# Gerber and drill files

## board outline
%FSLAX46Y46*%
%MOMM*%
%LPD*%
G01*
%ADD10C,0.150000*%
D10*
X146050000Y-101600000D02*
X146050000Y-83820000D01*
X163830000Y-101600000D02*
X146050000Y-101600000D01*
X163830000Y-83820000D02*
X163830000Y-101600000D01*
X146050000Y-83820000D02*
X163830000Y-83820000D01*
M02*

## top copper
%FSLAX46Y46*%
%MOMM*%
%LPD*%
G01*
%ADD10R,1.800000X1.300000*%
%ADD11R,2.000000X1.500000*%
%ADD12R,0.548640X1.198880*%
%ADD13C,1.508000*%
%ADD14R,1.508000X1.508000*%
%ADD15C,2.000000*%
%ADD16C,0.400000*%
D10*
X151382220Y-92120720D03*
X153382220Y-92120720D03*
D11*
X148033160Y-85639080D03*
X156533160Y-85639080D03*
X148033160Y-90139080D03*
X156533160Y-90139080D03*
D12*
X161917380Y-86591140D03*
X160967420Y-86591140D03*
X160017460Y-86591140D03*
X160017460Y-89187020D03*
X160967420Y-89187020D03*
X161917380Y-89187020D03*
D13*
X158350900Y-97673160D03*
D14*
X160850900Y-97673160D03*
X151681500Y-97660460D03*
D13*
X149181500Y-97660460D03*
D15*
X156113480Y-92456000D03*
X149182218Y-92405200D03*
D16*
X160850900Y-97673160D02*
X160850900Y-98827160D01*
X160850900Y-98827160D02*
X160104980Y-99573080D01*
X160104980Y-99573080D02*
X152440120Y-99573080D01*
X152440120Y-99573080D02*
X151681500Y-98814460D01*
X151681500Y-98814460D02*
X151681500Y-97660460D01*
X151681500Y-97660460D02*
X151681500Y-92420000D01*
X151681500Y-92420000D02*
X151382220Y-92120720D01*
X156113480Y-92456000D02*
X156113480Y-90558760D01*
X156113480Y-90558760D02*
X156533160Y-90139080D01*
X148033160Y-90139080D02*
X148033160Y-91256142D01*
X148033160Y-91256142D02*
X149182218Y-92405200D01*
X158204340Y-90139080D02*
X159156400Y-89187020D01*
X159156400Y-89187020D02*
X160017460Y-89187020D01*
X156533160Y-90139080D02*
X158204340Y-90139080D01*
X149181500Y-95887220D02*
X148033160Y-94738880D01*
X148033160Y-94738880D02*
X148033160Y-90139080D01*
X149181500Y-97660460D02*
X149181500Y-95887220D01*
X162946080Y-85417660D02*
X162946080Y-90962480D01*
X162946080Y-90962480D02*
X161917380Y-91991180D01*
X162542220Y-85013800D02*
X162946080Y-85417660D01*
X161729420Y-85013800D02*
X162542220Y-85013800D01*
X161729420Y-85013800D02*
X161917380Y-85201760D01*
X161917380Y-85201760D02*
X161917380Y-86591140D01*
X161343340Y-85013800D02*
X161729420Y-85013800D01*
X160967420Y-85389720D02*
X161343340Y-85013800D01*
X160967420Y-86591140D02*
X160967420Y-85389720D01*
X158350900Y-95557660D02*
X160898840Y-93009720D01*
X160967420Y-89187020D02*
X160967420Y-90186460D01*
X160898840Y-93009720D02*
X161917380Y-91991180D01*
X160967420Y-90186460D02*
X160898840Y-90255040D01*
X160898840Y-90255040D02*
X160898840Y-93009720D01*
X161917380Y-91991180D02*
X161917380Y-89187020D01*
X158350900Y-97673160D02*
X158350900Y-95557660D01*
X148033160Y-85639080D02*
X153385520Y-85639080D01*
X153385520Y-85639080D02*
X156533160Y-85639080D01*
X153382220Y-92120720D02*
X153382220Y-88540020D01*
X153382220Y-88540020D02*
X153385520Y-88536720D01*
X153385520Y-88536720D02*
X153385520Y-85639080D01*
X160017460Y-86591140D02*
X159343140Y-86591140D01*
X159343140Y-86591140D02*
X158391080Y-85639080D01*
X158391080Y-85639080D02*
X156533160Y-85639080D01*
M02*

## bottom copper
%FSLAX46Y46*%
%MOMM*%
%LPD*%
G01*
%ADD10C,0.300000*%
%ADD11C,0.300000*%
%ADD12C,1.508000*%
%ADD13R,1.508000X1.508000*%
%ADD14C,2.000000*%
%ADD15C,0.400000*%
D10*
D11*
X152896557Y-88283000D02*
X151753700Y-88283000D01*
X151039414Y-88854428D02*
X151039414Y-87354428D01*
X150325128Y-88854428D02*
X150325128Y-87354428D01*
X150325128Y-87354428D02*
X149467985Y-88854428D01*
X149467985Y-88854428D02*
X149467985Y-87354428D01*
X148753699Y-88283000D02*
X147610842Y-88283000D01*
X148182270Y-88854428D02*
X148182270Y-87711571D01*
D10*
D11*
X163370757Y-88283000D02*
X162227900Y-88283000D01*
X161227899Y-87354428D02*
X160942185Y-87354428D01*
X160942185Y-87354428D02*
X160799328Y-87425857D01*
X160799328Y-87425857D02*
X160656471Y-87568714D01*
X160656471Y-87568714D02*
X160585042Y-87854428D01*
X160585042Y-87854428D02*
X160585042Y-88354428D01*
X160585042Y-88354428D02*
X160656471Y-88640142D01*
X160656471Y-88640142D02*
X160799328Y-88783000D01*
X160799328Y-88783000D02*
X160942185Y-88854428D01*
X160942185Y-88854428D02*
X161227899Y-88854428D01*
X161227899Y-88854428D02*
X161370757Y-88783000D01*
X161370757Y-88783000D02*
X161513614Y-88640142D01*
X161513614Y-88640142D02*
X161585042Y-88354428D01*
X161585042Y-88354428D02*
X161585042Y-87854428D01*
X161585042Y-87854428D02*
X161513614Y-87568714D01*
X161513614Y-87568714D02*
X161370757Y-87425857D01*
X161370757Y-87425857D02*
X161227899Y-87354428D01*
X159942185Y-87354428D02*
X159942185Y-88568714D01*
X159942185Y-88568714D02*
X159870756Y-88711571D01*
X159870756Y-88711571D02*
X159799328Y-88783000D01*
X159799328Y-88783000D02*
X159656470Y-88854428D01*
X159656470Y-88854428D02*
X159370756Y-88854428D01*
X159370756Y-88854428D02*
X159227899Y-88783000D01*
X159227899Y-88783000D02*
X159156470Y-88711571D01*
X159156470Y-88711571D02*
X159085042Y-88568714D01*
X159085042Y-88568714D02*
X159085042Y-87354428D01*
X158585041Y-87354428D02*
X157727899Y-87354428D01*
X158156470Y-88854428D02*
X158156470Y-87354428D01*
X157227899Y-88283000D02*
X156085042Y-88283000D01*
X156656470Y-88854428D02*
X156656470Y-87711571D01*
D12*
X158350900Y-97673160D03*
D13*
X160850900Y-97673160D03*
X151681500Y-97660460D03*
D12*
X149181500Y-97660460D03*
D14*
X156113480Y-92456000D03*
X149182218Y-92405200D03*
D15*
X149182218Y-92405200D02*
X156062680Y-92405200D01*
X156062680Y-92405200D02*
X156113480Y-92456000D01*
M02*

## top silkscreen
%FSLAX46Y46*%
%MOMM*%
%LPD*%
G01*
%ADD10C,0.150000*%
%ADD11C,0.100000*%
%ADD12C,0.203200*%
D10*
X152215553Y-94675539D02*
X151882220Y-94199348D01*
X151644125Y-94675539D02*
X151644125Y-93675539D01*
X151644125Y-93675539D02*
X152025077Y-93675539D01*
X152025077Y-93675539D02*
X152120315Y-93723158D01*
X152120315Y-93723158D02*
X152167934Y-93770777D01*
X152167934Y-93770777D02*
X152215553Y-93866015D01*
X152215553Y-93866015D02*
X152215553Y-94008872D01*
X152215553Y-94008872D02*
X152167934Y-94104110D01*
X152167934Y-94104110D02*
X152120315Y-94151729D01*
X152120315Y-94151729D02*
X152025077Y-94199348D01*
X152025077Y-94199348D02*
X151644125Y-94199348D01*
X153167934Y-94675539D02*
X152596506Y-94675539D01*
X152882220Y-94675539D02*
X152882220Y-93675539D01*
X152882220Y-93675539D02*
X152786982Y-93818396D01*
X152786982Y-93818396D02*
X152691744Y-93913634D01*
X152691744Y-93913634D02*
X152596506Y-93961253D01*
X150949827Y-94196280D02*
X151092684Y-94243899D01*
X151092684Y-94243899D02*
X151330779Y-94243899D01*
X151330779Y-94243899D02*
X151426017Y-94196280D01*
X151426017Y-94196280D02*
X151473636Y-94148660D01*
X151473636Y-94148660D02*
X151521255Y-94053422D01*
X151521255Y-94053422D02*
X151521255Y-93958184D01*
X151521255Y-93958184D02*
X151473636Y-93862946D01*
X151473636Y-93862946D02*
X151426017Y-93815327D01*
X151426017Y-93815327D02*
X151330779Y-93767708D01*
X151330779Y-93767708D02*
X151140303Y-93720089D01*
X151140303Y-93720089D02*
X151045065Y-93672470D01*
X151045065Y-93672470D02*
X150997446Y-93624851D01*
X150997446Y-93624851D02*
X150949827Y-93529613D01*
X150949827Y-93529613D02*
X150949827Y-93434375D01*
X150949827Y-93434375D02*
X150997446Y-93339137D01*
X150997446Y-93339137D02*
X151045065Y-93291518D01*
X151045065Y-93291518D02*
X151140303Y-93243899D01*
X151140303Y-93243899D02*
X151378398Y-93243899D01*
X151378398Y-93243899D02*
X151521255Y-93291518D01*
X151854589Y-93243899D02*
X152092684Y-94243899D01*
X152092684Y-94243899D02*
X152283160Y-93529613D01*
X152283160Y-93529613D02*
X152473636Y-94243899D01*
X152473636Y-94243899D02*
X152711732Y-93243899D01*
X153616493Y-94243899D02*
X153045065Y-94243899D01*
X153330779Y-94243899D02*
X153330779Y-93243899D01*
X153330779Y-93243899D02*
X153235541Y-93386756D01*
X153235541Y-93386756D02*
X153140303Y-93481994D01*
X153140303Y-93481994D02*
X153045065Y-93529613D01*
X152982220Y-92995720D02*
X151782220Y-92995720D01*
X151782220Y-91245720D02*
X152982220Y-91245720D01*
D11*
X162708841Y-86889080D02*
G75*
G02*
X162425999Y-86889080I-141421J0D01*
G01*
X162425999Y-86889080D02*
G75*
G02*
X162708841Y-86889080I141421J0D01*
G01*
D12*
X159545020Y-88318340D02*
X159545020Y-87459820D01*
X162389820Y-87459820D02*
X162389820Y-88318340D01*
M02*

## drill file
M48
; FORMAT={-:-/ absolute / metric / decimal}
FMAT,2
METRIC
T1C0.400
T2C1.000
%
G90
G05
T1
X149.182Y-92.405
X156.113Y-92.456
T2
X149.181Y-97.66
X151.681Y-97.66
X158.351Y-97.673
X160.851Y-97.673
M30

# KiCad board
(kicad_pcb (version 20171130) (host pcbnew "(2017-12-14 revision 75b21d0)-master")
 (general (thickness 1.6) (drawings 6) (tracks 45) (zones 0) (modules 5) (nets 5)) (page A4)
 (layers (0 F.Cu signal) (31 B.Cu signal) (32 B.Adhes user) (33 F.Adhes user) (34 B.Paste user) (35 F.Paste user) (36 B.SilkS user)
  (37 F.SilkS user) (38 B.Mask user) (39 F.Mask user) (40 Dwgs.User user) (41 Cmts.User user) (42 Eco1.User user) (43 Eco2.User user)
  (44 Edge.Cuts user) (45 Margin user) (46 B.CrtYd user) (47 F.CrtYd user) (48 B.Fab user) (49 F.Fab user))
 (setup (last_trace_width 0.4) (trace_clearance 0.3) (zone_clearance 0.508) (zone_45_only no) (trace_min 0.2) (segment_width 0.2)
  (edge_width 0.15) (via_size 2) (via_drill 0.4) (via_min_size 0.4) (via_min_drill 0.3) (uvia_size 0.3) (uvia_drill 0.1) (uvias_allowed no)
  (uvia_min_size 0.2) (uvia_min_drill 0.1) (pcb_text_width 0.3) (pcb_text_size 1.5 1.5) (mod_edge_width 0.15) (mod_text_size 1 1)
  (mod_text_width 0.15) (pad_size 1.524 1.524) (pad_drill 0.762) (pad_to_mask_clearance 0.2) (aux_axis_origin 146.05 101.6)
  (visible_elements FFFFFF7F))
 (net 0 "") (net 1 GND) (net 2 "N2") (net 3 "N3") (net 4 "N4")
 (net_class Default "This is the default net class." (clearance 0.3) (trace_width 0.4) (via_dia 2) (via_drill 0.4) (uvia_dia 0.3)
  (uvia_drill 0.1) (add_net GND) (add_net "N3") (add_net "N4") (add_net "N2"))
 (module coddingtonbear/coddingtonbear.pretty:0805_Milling (layer F.Cu) (at 152.38222 92.12072 180)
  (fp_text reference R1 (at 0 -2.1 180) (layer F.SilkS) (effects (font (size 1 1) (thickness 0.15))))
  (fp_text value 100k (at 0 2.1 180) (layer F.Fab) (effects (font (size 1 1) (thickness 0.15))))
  (fp_line (start -0.6 -0.875) (end 0.6 -0.875) (layer F.SilkS) (width 0.15))
  (fp_line (start 0.6 0.875) (end -0.6 0.875) (layer F.SilkS) (width 0.15))
  (pad 2 smd rect (at 1 0 180) (size 1.8 1.3) (layers F.Cu F.Paste F.Mask) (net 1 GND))
  (pad 1 smd rect (at -1 0 180) (size 1.8 1.3) (layers F.Cu F.Paste F.Mask) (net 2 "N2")))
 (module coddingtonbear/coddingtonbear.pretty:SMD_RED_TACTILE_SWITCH (layer F.Cu) (at 152.28316 87.88908)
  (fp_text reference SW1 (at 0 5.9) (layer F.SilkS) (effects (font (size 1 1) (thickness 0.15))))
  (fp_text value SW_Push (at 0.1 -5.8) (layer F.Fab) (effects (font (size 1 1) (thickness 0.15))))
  (pad 1 smd rect (at -4.25 -2.25) (size 2 1.5) (layers F.Cu F.Paste F.Mask) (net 2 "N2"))
  (pad 1 smd rect (at 4.25 -2.25) (size 2 1.5) (layers F.Cu F.Paste F.Mask) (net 2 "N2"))
  (pad 2 smd rect (at -4.25 2.25) (size 2 1.5) (layers F.Cu F.Paste F.Mask) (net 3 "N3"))
  (pad 2 smd rect (at 4.25 2.25) (size 2 1.5) (layers F.Cu F.Paste F.Mask) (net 3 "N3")))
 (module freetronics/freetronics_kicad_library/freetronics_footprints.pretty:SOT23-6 (layer F.Cu) (at 160.96742 87.88908 180)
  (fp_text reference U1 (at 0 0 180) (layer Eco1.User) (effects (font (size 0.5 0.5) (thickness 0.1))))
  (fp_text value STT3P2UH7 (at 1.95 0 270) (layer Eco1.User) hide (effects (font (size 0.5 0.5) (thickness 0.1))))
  (fp_circle (center -1.6 1) (end -1.5 0.9) (layer F.SilkS) (width 0.1))
  (fp_line (start 1.4224 -0.42926) (end 1.4224 0.42926) (layer F.SilkS) (width 0.2032))
  (fp_line (start -1.4224 0.42926) (end -1.4224 -0.42926) (layer F.SilkS) (width 0.2032))
  (pad 1 smd rect (at -0.94996 1.29794 180) (size 0.54864 1.19888) (layers F.Cu F.Paste F.Mask) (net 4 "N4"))
  (pad 2 smd rect (at 0 1.29794 180) (size 0.54864 1.19888) (layers F.Cu F.Paste F.Mask) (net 4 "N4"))
  (pad 3 smd rect (at 0.94996 1.29794 180) (size 0.54864 1.19888) (layers F.Cu F.Paste F.Mask) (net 2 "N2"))
  (pad 4 smd rect (at 0.94996 -1.29794 180) (size 0.54864 1.19888) (layers F.Cu F.Paste F.Mask) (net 3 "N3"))
  (pad 5 smd rect (at 0 -1.29794 180) (size 0.54864 1.19888) (layers F.Cu F.Paste F.Mask) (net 4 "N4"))
  (pad 6 smd rect (at -0.94996 -1.29794 180) (size 0.54864 1.19888) (layers F.Cu F.Paste F.Mask) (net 4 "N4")))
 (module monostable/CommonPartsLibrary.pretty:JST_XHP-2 (layer B.Cu) (at 159.6009 97.67316) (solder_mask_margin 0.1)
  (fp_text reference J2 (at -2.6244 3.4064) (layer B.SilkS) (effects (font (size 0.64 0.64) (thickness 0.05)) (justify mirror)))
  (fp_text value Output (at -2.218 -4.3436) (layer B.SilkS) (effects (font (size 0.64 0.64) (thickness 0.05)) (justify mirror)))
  (pad 2 thru_hole circle (at -1.25 0 270) (size 1.508 1.508) (drill 1) (layers *.Cu *.Mask B.SilkS) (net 4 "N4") (solder_mask_margin 0.2))
  (pad 1 thru_hole rect (at 1.25 0 270) (size 1.508 1.508) (drill 1) (layers *.Cu *.Mask B.SilkS) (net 1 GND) (solder_mask_margin 0.2)))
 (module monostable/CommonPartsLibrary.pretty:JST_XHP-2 (layer B.Cu) (at 150.4315 97.66046) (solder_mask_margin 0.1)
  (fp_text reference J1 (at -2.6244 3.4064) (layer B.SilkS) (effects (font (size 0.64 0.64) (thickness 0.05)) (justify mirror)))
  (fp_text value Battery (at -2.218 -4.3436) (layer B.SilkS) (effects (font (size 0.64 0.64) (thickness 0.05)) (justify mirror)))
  (pad 1 thru_hole rect (at 1.25 0 270) (size 1.508 1.508) (drill 1) (layers *.Cu *.Mask B.SilkS) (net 1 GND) (solder_mask_margin 0.2))
  (pad 2 thru_hole circle (at -1.25 0 270) (size 1.508 1.508) (drill 1) (layers *.Cu *.Mask B.SilkS) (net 3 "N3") (solder_mask_margin 0.2)))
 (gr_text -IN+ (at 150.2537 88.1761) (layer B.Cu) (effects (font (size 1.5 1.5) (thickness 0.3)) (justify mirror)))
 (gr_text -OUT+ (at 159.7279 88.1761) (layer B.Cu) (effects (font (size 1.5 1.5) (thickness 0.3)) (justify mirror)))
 (gr_line (start 146.05 101.6) (end 146.05 83.82) (layer Edge.Cuts) (width 0.15))
 (gr_line (start 163.83 101.6) (end 146.05 101.6) (layer Edge.Cuts) (width 0.15))
 (gr_line (start 163.83 83.82) (end 163.83 101.6) (layer Edge.Cuts) (width 0.15))
 (gr_line (start 146.05 83.82) (end 163.83 83.82) (layer Edge.Cuts) (width 0.15))
 (segment (start 160.8509 97.67316) (end 160.8509 98.82716) (width 0.4) (layer F.Cu) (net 1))
 (segment (start 160.8509 98.82716) (end 160.10498 99.57308) (width 0.4) (layer F.Cu) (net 1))
 (segment (start 160.10498 99.57308) (end 152.44012 99.57308) (width 0.4) (layer F.Cu) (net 1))
 (segment (start 152.44012 99.57308) (end 151.6815 98.81446) (width 0.4) (layer F.Cu) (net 1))
 (segment (start 151.6815 98.81446) (end 151.6815 97.66046) (width 0.4) (layer F.Cu) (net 1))
 (segment (start 151.6815 97.66046) (end 151.6815 92.42) (width 0.4) (layer F.Cu) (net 1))
 (segment (start 151.6815 92.42) (end 151.38222 92.12072) (width 0.4) (layer F.Cu) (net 1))
 (segment (start 156.11348 92.456) (end 156.11348 90.55876) (width 0.4) (layer F.Cu) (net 3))
 (segment (start 156.11348 90.55876) (end 156.53316 90.13908) (width 0.4) (layer F.Cu) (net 3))
 (segment (start 149.182218 92.4052) (end 156.06268 92.4052) (width 0.4) (layer B.Cu) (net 3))
 (segment (start 156.06268 92.4052) (end 156.11348 92.456) (width 0.4) (layer B.Cu) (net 3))
 (via (at 156.11348 92.456) (size 2) (drill 0.4) (layers F.Cu B.Cu) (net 3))
 (segment (start 148.03316 90.13908) (end 148.03316 91.256142) (width 0.4) (layer F.Cu) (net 3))
 (segment (start 148.03316 91.256142) (end 149.182218 92.4052) (width 0.4) (layer F.Cu) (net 3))
 (via (at 149.182218 92.4052) (size 2) (drill 0.4) (layers F.Cu B.Cu) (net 3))
 (segment (start 158.20434 90.13908) (end 159.1564 89.18702) (width 0.4) (layer F.Cu) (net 3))
 (segment (start 159.1564 89.18702) (end 160.01746 89.18702) (width 0.4) (layer F.Cu) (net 3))
 (segment (start 156.53316 90.13908) (end 158.20434 90.13908) (width 0.4) (layer F.Cu) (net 3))
 (segment (start 149.1815 95.88722) (end 148.03316 94.73888) (width 0.4) (layer F.Cu) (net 3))
 (segment (start 148.03316 94.73888) (end 148.03316 90.13908) (width 0.4) (layer F.Cu) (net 3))
 (segment (start 149.1815 97.66046) (end 149.1815 95.88722) (width 0.4) (layer F.Cu) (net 3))
 (segment (start 162.94608 85.41766) (end 162.94608 90.96248) (width 0.4) (layer F.Cu) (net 4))
 (segment (start 162.94608 90.96248) (end 161.91738 91.99118) (width 0.4) (layer F.Cu) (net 4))
 (segment (start 162.54222 85.0138) (end 162.94608 85.41766) (width 0.4) (layer F.Cu) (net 4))
 (segment (start 161.72942 85.0138) (end 162.54222 85.0138) (width 0.4) (layer F.Cu) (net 4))
 (segment (start 161.72942 85.0138) (end 161.91738 85.20176) (width 0.4) (layer F.Cu) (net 4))
 (segment (start 161.91738 85.20176) (end 161.91738 86.59114) (width 0.4) (layer F.Cu) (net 4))
 (segment (start 161.34334 85.0138) (end 161.72942 85.0138) (width 0.4) (layer F.Cu) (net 4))
 (segment (start 160.96742 85.38972) (end 161.34334 85.0138) (width 0.4) (layer F.Cu) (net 4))
 (segment (start 160.96742 86.59114) (end 160.96742 85.38972) (width 0.4) (layer F.Cu) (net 4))
 (segment (start 158.3509 95.55766) (end 160.89884 93.00972) (width 0.4) (layer F.Cu) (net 4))
 (segment (start 160.96742 89.18702) (end 160.96742 90.18646) (width 0.4) (layer F.Cu) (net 4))
 (segment (start 160.89884 93.00972) (end 161.91738 91.99118) (width 0.4) (layer F.Cu) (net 4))
 (segment (start 160.96742 90.18646) (end 160.89884 90.25504) (width 0.4) (layer F.Cu) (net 4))
 (segment (start 160.89884 90.25504) (end 160.89884 93.00972) (width 0.4) (layer F.Cu) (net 4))
 (segment (start 161.91738 91.99118) (end 161.91738 89.18702) (width 0.4) (layer F.Cu) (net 4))
 (segment (start 158.3509 97.67316) (end 158.3509 95.55766) (width 0.4) (layer F.Cu) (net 4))
 (segment (start 148.03316 85.63908) (end 153.38552 85.63908) (width 0.4) (layer F.Cu) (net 2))
 (segment (start 153.38552 85.63908) (end 156.53316 85.63908) (width 0.4) (layer F.Cu) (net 2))
 (segment (start 153.38222 92.12072) (end 153.38222 88.54002) (width 0.4) (layer F.Cu) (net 2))
 (segment (start 153.38222 88.54002) (end 153.38552 88.53672) (width 0.4) (layer F.Cu) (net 2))
 (segment (start 153.38552 88.53672) (end 153.38552 85.63908) (width 0.4) (layer F.Cu) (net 2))
 (segment (start 160.01746 86.59114) (end 159.34314 86.59114) (width 0.4) (layer F.Cu) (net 2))
 (segment (start 159.34314 86.59114) (end 158.39108 85.63908) (width 0.4) (layer F.Cu) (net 2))
 (segment (start 158.39108 85.63908) (end 156.53316 85.63908) (width 0.4) (layer F.Cu) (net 2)))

